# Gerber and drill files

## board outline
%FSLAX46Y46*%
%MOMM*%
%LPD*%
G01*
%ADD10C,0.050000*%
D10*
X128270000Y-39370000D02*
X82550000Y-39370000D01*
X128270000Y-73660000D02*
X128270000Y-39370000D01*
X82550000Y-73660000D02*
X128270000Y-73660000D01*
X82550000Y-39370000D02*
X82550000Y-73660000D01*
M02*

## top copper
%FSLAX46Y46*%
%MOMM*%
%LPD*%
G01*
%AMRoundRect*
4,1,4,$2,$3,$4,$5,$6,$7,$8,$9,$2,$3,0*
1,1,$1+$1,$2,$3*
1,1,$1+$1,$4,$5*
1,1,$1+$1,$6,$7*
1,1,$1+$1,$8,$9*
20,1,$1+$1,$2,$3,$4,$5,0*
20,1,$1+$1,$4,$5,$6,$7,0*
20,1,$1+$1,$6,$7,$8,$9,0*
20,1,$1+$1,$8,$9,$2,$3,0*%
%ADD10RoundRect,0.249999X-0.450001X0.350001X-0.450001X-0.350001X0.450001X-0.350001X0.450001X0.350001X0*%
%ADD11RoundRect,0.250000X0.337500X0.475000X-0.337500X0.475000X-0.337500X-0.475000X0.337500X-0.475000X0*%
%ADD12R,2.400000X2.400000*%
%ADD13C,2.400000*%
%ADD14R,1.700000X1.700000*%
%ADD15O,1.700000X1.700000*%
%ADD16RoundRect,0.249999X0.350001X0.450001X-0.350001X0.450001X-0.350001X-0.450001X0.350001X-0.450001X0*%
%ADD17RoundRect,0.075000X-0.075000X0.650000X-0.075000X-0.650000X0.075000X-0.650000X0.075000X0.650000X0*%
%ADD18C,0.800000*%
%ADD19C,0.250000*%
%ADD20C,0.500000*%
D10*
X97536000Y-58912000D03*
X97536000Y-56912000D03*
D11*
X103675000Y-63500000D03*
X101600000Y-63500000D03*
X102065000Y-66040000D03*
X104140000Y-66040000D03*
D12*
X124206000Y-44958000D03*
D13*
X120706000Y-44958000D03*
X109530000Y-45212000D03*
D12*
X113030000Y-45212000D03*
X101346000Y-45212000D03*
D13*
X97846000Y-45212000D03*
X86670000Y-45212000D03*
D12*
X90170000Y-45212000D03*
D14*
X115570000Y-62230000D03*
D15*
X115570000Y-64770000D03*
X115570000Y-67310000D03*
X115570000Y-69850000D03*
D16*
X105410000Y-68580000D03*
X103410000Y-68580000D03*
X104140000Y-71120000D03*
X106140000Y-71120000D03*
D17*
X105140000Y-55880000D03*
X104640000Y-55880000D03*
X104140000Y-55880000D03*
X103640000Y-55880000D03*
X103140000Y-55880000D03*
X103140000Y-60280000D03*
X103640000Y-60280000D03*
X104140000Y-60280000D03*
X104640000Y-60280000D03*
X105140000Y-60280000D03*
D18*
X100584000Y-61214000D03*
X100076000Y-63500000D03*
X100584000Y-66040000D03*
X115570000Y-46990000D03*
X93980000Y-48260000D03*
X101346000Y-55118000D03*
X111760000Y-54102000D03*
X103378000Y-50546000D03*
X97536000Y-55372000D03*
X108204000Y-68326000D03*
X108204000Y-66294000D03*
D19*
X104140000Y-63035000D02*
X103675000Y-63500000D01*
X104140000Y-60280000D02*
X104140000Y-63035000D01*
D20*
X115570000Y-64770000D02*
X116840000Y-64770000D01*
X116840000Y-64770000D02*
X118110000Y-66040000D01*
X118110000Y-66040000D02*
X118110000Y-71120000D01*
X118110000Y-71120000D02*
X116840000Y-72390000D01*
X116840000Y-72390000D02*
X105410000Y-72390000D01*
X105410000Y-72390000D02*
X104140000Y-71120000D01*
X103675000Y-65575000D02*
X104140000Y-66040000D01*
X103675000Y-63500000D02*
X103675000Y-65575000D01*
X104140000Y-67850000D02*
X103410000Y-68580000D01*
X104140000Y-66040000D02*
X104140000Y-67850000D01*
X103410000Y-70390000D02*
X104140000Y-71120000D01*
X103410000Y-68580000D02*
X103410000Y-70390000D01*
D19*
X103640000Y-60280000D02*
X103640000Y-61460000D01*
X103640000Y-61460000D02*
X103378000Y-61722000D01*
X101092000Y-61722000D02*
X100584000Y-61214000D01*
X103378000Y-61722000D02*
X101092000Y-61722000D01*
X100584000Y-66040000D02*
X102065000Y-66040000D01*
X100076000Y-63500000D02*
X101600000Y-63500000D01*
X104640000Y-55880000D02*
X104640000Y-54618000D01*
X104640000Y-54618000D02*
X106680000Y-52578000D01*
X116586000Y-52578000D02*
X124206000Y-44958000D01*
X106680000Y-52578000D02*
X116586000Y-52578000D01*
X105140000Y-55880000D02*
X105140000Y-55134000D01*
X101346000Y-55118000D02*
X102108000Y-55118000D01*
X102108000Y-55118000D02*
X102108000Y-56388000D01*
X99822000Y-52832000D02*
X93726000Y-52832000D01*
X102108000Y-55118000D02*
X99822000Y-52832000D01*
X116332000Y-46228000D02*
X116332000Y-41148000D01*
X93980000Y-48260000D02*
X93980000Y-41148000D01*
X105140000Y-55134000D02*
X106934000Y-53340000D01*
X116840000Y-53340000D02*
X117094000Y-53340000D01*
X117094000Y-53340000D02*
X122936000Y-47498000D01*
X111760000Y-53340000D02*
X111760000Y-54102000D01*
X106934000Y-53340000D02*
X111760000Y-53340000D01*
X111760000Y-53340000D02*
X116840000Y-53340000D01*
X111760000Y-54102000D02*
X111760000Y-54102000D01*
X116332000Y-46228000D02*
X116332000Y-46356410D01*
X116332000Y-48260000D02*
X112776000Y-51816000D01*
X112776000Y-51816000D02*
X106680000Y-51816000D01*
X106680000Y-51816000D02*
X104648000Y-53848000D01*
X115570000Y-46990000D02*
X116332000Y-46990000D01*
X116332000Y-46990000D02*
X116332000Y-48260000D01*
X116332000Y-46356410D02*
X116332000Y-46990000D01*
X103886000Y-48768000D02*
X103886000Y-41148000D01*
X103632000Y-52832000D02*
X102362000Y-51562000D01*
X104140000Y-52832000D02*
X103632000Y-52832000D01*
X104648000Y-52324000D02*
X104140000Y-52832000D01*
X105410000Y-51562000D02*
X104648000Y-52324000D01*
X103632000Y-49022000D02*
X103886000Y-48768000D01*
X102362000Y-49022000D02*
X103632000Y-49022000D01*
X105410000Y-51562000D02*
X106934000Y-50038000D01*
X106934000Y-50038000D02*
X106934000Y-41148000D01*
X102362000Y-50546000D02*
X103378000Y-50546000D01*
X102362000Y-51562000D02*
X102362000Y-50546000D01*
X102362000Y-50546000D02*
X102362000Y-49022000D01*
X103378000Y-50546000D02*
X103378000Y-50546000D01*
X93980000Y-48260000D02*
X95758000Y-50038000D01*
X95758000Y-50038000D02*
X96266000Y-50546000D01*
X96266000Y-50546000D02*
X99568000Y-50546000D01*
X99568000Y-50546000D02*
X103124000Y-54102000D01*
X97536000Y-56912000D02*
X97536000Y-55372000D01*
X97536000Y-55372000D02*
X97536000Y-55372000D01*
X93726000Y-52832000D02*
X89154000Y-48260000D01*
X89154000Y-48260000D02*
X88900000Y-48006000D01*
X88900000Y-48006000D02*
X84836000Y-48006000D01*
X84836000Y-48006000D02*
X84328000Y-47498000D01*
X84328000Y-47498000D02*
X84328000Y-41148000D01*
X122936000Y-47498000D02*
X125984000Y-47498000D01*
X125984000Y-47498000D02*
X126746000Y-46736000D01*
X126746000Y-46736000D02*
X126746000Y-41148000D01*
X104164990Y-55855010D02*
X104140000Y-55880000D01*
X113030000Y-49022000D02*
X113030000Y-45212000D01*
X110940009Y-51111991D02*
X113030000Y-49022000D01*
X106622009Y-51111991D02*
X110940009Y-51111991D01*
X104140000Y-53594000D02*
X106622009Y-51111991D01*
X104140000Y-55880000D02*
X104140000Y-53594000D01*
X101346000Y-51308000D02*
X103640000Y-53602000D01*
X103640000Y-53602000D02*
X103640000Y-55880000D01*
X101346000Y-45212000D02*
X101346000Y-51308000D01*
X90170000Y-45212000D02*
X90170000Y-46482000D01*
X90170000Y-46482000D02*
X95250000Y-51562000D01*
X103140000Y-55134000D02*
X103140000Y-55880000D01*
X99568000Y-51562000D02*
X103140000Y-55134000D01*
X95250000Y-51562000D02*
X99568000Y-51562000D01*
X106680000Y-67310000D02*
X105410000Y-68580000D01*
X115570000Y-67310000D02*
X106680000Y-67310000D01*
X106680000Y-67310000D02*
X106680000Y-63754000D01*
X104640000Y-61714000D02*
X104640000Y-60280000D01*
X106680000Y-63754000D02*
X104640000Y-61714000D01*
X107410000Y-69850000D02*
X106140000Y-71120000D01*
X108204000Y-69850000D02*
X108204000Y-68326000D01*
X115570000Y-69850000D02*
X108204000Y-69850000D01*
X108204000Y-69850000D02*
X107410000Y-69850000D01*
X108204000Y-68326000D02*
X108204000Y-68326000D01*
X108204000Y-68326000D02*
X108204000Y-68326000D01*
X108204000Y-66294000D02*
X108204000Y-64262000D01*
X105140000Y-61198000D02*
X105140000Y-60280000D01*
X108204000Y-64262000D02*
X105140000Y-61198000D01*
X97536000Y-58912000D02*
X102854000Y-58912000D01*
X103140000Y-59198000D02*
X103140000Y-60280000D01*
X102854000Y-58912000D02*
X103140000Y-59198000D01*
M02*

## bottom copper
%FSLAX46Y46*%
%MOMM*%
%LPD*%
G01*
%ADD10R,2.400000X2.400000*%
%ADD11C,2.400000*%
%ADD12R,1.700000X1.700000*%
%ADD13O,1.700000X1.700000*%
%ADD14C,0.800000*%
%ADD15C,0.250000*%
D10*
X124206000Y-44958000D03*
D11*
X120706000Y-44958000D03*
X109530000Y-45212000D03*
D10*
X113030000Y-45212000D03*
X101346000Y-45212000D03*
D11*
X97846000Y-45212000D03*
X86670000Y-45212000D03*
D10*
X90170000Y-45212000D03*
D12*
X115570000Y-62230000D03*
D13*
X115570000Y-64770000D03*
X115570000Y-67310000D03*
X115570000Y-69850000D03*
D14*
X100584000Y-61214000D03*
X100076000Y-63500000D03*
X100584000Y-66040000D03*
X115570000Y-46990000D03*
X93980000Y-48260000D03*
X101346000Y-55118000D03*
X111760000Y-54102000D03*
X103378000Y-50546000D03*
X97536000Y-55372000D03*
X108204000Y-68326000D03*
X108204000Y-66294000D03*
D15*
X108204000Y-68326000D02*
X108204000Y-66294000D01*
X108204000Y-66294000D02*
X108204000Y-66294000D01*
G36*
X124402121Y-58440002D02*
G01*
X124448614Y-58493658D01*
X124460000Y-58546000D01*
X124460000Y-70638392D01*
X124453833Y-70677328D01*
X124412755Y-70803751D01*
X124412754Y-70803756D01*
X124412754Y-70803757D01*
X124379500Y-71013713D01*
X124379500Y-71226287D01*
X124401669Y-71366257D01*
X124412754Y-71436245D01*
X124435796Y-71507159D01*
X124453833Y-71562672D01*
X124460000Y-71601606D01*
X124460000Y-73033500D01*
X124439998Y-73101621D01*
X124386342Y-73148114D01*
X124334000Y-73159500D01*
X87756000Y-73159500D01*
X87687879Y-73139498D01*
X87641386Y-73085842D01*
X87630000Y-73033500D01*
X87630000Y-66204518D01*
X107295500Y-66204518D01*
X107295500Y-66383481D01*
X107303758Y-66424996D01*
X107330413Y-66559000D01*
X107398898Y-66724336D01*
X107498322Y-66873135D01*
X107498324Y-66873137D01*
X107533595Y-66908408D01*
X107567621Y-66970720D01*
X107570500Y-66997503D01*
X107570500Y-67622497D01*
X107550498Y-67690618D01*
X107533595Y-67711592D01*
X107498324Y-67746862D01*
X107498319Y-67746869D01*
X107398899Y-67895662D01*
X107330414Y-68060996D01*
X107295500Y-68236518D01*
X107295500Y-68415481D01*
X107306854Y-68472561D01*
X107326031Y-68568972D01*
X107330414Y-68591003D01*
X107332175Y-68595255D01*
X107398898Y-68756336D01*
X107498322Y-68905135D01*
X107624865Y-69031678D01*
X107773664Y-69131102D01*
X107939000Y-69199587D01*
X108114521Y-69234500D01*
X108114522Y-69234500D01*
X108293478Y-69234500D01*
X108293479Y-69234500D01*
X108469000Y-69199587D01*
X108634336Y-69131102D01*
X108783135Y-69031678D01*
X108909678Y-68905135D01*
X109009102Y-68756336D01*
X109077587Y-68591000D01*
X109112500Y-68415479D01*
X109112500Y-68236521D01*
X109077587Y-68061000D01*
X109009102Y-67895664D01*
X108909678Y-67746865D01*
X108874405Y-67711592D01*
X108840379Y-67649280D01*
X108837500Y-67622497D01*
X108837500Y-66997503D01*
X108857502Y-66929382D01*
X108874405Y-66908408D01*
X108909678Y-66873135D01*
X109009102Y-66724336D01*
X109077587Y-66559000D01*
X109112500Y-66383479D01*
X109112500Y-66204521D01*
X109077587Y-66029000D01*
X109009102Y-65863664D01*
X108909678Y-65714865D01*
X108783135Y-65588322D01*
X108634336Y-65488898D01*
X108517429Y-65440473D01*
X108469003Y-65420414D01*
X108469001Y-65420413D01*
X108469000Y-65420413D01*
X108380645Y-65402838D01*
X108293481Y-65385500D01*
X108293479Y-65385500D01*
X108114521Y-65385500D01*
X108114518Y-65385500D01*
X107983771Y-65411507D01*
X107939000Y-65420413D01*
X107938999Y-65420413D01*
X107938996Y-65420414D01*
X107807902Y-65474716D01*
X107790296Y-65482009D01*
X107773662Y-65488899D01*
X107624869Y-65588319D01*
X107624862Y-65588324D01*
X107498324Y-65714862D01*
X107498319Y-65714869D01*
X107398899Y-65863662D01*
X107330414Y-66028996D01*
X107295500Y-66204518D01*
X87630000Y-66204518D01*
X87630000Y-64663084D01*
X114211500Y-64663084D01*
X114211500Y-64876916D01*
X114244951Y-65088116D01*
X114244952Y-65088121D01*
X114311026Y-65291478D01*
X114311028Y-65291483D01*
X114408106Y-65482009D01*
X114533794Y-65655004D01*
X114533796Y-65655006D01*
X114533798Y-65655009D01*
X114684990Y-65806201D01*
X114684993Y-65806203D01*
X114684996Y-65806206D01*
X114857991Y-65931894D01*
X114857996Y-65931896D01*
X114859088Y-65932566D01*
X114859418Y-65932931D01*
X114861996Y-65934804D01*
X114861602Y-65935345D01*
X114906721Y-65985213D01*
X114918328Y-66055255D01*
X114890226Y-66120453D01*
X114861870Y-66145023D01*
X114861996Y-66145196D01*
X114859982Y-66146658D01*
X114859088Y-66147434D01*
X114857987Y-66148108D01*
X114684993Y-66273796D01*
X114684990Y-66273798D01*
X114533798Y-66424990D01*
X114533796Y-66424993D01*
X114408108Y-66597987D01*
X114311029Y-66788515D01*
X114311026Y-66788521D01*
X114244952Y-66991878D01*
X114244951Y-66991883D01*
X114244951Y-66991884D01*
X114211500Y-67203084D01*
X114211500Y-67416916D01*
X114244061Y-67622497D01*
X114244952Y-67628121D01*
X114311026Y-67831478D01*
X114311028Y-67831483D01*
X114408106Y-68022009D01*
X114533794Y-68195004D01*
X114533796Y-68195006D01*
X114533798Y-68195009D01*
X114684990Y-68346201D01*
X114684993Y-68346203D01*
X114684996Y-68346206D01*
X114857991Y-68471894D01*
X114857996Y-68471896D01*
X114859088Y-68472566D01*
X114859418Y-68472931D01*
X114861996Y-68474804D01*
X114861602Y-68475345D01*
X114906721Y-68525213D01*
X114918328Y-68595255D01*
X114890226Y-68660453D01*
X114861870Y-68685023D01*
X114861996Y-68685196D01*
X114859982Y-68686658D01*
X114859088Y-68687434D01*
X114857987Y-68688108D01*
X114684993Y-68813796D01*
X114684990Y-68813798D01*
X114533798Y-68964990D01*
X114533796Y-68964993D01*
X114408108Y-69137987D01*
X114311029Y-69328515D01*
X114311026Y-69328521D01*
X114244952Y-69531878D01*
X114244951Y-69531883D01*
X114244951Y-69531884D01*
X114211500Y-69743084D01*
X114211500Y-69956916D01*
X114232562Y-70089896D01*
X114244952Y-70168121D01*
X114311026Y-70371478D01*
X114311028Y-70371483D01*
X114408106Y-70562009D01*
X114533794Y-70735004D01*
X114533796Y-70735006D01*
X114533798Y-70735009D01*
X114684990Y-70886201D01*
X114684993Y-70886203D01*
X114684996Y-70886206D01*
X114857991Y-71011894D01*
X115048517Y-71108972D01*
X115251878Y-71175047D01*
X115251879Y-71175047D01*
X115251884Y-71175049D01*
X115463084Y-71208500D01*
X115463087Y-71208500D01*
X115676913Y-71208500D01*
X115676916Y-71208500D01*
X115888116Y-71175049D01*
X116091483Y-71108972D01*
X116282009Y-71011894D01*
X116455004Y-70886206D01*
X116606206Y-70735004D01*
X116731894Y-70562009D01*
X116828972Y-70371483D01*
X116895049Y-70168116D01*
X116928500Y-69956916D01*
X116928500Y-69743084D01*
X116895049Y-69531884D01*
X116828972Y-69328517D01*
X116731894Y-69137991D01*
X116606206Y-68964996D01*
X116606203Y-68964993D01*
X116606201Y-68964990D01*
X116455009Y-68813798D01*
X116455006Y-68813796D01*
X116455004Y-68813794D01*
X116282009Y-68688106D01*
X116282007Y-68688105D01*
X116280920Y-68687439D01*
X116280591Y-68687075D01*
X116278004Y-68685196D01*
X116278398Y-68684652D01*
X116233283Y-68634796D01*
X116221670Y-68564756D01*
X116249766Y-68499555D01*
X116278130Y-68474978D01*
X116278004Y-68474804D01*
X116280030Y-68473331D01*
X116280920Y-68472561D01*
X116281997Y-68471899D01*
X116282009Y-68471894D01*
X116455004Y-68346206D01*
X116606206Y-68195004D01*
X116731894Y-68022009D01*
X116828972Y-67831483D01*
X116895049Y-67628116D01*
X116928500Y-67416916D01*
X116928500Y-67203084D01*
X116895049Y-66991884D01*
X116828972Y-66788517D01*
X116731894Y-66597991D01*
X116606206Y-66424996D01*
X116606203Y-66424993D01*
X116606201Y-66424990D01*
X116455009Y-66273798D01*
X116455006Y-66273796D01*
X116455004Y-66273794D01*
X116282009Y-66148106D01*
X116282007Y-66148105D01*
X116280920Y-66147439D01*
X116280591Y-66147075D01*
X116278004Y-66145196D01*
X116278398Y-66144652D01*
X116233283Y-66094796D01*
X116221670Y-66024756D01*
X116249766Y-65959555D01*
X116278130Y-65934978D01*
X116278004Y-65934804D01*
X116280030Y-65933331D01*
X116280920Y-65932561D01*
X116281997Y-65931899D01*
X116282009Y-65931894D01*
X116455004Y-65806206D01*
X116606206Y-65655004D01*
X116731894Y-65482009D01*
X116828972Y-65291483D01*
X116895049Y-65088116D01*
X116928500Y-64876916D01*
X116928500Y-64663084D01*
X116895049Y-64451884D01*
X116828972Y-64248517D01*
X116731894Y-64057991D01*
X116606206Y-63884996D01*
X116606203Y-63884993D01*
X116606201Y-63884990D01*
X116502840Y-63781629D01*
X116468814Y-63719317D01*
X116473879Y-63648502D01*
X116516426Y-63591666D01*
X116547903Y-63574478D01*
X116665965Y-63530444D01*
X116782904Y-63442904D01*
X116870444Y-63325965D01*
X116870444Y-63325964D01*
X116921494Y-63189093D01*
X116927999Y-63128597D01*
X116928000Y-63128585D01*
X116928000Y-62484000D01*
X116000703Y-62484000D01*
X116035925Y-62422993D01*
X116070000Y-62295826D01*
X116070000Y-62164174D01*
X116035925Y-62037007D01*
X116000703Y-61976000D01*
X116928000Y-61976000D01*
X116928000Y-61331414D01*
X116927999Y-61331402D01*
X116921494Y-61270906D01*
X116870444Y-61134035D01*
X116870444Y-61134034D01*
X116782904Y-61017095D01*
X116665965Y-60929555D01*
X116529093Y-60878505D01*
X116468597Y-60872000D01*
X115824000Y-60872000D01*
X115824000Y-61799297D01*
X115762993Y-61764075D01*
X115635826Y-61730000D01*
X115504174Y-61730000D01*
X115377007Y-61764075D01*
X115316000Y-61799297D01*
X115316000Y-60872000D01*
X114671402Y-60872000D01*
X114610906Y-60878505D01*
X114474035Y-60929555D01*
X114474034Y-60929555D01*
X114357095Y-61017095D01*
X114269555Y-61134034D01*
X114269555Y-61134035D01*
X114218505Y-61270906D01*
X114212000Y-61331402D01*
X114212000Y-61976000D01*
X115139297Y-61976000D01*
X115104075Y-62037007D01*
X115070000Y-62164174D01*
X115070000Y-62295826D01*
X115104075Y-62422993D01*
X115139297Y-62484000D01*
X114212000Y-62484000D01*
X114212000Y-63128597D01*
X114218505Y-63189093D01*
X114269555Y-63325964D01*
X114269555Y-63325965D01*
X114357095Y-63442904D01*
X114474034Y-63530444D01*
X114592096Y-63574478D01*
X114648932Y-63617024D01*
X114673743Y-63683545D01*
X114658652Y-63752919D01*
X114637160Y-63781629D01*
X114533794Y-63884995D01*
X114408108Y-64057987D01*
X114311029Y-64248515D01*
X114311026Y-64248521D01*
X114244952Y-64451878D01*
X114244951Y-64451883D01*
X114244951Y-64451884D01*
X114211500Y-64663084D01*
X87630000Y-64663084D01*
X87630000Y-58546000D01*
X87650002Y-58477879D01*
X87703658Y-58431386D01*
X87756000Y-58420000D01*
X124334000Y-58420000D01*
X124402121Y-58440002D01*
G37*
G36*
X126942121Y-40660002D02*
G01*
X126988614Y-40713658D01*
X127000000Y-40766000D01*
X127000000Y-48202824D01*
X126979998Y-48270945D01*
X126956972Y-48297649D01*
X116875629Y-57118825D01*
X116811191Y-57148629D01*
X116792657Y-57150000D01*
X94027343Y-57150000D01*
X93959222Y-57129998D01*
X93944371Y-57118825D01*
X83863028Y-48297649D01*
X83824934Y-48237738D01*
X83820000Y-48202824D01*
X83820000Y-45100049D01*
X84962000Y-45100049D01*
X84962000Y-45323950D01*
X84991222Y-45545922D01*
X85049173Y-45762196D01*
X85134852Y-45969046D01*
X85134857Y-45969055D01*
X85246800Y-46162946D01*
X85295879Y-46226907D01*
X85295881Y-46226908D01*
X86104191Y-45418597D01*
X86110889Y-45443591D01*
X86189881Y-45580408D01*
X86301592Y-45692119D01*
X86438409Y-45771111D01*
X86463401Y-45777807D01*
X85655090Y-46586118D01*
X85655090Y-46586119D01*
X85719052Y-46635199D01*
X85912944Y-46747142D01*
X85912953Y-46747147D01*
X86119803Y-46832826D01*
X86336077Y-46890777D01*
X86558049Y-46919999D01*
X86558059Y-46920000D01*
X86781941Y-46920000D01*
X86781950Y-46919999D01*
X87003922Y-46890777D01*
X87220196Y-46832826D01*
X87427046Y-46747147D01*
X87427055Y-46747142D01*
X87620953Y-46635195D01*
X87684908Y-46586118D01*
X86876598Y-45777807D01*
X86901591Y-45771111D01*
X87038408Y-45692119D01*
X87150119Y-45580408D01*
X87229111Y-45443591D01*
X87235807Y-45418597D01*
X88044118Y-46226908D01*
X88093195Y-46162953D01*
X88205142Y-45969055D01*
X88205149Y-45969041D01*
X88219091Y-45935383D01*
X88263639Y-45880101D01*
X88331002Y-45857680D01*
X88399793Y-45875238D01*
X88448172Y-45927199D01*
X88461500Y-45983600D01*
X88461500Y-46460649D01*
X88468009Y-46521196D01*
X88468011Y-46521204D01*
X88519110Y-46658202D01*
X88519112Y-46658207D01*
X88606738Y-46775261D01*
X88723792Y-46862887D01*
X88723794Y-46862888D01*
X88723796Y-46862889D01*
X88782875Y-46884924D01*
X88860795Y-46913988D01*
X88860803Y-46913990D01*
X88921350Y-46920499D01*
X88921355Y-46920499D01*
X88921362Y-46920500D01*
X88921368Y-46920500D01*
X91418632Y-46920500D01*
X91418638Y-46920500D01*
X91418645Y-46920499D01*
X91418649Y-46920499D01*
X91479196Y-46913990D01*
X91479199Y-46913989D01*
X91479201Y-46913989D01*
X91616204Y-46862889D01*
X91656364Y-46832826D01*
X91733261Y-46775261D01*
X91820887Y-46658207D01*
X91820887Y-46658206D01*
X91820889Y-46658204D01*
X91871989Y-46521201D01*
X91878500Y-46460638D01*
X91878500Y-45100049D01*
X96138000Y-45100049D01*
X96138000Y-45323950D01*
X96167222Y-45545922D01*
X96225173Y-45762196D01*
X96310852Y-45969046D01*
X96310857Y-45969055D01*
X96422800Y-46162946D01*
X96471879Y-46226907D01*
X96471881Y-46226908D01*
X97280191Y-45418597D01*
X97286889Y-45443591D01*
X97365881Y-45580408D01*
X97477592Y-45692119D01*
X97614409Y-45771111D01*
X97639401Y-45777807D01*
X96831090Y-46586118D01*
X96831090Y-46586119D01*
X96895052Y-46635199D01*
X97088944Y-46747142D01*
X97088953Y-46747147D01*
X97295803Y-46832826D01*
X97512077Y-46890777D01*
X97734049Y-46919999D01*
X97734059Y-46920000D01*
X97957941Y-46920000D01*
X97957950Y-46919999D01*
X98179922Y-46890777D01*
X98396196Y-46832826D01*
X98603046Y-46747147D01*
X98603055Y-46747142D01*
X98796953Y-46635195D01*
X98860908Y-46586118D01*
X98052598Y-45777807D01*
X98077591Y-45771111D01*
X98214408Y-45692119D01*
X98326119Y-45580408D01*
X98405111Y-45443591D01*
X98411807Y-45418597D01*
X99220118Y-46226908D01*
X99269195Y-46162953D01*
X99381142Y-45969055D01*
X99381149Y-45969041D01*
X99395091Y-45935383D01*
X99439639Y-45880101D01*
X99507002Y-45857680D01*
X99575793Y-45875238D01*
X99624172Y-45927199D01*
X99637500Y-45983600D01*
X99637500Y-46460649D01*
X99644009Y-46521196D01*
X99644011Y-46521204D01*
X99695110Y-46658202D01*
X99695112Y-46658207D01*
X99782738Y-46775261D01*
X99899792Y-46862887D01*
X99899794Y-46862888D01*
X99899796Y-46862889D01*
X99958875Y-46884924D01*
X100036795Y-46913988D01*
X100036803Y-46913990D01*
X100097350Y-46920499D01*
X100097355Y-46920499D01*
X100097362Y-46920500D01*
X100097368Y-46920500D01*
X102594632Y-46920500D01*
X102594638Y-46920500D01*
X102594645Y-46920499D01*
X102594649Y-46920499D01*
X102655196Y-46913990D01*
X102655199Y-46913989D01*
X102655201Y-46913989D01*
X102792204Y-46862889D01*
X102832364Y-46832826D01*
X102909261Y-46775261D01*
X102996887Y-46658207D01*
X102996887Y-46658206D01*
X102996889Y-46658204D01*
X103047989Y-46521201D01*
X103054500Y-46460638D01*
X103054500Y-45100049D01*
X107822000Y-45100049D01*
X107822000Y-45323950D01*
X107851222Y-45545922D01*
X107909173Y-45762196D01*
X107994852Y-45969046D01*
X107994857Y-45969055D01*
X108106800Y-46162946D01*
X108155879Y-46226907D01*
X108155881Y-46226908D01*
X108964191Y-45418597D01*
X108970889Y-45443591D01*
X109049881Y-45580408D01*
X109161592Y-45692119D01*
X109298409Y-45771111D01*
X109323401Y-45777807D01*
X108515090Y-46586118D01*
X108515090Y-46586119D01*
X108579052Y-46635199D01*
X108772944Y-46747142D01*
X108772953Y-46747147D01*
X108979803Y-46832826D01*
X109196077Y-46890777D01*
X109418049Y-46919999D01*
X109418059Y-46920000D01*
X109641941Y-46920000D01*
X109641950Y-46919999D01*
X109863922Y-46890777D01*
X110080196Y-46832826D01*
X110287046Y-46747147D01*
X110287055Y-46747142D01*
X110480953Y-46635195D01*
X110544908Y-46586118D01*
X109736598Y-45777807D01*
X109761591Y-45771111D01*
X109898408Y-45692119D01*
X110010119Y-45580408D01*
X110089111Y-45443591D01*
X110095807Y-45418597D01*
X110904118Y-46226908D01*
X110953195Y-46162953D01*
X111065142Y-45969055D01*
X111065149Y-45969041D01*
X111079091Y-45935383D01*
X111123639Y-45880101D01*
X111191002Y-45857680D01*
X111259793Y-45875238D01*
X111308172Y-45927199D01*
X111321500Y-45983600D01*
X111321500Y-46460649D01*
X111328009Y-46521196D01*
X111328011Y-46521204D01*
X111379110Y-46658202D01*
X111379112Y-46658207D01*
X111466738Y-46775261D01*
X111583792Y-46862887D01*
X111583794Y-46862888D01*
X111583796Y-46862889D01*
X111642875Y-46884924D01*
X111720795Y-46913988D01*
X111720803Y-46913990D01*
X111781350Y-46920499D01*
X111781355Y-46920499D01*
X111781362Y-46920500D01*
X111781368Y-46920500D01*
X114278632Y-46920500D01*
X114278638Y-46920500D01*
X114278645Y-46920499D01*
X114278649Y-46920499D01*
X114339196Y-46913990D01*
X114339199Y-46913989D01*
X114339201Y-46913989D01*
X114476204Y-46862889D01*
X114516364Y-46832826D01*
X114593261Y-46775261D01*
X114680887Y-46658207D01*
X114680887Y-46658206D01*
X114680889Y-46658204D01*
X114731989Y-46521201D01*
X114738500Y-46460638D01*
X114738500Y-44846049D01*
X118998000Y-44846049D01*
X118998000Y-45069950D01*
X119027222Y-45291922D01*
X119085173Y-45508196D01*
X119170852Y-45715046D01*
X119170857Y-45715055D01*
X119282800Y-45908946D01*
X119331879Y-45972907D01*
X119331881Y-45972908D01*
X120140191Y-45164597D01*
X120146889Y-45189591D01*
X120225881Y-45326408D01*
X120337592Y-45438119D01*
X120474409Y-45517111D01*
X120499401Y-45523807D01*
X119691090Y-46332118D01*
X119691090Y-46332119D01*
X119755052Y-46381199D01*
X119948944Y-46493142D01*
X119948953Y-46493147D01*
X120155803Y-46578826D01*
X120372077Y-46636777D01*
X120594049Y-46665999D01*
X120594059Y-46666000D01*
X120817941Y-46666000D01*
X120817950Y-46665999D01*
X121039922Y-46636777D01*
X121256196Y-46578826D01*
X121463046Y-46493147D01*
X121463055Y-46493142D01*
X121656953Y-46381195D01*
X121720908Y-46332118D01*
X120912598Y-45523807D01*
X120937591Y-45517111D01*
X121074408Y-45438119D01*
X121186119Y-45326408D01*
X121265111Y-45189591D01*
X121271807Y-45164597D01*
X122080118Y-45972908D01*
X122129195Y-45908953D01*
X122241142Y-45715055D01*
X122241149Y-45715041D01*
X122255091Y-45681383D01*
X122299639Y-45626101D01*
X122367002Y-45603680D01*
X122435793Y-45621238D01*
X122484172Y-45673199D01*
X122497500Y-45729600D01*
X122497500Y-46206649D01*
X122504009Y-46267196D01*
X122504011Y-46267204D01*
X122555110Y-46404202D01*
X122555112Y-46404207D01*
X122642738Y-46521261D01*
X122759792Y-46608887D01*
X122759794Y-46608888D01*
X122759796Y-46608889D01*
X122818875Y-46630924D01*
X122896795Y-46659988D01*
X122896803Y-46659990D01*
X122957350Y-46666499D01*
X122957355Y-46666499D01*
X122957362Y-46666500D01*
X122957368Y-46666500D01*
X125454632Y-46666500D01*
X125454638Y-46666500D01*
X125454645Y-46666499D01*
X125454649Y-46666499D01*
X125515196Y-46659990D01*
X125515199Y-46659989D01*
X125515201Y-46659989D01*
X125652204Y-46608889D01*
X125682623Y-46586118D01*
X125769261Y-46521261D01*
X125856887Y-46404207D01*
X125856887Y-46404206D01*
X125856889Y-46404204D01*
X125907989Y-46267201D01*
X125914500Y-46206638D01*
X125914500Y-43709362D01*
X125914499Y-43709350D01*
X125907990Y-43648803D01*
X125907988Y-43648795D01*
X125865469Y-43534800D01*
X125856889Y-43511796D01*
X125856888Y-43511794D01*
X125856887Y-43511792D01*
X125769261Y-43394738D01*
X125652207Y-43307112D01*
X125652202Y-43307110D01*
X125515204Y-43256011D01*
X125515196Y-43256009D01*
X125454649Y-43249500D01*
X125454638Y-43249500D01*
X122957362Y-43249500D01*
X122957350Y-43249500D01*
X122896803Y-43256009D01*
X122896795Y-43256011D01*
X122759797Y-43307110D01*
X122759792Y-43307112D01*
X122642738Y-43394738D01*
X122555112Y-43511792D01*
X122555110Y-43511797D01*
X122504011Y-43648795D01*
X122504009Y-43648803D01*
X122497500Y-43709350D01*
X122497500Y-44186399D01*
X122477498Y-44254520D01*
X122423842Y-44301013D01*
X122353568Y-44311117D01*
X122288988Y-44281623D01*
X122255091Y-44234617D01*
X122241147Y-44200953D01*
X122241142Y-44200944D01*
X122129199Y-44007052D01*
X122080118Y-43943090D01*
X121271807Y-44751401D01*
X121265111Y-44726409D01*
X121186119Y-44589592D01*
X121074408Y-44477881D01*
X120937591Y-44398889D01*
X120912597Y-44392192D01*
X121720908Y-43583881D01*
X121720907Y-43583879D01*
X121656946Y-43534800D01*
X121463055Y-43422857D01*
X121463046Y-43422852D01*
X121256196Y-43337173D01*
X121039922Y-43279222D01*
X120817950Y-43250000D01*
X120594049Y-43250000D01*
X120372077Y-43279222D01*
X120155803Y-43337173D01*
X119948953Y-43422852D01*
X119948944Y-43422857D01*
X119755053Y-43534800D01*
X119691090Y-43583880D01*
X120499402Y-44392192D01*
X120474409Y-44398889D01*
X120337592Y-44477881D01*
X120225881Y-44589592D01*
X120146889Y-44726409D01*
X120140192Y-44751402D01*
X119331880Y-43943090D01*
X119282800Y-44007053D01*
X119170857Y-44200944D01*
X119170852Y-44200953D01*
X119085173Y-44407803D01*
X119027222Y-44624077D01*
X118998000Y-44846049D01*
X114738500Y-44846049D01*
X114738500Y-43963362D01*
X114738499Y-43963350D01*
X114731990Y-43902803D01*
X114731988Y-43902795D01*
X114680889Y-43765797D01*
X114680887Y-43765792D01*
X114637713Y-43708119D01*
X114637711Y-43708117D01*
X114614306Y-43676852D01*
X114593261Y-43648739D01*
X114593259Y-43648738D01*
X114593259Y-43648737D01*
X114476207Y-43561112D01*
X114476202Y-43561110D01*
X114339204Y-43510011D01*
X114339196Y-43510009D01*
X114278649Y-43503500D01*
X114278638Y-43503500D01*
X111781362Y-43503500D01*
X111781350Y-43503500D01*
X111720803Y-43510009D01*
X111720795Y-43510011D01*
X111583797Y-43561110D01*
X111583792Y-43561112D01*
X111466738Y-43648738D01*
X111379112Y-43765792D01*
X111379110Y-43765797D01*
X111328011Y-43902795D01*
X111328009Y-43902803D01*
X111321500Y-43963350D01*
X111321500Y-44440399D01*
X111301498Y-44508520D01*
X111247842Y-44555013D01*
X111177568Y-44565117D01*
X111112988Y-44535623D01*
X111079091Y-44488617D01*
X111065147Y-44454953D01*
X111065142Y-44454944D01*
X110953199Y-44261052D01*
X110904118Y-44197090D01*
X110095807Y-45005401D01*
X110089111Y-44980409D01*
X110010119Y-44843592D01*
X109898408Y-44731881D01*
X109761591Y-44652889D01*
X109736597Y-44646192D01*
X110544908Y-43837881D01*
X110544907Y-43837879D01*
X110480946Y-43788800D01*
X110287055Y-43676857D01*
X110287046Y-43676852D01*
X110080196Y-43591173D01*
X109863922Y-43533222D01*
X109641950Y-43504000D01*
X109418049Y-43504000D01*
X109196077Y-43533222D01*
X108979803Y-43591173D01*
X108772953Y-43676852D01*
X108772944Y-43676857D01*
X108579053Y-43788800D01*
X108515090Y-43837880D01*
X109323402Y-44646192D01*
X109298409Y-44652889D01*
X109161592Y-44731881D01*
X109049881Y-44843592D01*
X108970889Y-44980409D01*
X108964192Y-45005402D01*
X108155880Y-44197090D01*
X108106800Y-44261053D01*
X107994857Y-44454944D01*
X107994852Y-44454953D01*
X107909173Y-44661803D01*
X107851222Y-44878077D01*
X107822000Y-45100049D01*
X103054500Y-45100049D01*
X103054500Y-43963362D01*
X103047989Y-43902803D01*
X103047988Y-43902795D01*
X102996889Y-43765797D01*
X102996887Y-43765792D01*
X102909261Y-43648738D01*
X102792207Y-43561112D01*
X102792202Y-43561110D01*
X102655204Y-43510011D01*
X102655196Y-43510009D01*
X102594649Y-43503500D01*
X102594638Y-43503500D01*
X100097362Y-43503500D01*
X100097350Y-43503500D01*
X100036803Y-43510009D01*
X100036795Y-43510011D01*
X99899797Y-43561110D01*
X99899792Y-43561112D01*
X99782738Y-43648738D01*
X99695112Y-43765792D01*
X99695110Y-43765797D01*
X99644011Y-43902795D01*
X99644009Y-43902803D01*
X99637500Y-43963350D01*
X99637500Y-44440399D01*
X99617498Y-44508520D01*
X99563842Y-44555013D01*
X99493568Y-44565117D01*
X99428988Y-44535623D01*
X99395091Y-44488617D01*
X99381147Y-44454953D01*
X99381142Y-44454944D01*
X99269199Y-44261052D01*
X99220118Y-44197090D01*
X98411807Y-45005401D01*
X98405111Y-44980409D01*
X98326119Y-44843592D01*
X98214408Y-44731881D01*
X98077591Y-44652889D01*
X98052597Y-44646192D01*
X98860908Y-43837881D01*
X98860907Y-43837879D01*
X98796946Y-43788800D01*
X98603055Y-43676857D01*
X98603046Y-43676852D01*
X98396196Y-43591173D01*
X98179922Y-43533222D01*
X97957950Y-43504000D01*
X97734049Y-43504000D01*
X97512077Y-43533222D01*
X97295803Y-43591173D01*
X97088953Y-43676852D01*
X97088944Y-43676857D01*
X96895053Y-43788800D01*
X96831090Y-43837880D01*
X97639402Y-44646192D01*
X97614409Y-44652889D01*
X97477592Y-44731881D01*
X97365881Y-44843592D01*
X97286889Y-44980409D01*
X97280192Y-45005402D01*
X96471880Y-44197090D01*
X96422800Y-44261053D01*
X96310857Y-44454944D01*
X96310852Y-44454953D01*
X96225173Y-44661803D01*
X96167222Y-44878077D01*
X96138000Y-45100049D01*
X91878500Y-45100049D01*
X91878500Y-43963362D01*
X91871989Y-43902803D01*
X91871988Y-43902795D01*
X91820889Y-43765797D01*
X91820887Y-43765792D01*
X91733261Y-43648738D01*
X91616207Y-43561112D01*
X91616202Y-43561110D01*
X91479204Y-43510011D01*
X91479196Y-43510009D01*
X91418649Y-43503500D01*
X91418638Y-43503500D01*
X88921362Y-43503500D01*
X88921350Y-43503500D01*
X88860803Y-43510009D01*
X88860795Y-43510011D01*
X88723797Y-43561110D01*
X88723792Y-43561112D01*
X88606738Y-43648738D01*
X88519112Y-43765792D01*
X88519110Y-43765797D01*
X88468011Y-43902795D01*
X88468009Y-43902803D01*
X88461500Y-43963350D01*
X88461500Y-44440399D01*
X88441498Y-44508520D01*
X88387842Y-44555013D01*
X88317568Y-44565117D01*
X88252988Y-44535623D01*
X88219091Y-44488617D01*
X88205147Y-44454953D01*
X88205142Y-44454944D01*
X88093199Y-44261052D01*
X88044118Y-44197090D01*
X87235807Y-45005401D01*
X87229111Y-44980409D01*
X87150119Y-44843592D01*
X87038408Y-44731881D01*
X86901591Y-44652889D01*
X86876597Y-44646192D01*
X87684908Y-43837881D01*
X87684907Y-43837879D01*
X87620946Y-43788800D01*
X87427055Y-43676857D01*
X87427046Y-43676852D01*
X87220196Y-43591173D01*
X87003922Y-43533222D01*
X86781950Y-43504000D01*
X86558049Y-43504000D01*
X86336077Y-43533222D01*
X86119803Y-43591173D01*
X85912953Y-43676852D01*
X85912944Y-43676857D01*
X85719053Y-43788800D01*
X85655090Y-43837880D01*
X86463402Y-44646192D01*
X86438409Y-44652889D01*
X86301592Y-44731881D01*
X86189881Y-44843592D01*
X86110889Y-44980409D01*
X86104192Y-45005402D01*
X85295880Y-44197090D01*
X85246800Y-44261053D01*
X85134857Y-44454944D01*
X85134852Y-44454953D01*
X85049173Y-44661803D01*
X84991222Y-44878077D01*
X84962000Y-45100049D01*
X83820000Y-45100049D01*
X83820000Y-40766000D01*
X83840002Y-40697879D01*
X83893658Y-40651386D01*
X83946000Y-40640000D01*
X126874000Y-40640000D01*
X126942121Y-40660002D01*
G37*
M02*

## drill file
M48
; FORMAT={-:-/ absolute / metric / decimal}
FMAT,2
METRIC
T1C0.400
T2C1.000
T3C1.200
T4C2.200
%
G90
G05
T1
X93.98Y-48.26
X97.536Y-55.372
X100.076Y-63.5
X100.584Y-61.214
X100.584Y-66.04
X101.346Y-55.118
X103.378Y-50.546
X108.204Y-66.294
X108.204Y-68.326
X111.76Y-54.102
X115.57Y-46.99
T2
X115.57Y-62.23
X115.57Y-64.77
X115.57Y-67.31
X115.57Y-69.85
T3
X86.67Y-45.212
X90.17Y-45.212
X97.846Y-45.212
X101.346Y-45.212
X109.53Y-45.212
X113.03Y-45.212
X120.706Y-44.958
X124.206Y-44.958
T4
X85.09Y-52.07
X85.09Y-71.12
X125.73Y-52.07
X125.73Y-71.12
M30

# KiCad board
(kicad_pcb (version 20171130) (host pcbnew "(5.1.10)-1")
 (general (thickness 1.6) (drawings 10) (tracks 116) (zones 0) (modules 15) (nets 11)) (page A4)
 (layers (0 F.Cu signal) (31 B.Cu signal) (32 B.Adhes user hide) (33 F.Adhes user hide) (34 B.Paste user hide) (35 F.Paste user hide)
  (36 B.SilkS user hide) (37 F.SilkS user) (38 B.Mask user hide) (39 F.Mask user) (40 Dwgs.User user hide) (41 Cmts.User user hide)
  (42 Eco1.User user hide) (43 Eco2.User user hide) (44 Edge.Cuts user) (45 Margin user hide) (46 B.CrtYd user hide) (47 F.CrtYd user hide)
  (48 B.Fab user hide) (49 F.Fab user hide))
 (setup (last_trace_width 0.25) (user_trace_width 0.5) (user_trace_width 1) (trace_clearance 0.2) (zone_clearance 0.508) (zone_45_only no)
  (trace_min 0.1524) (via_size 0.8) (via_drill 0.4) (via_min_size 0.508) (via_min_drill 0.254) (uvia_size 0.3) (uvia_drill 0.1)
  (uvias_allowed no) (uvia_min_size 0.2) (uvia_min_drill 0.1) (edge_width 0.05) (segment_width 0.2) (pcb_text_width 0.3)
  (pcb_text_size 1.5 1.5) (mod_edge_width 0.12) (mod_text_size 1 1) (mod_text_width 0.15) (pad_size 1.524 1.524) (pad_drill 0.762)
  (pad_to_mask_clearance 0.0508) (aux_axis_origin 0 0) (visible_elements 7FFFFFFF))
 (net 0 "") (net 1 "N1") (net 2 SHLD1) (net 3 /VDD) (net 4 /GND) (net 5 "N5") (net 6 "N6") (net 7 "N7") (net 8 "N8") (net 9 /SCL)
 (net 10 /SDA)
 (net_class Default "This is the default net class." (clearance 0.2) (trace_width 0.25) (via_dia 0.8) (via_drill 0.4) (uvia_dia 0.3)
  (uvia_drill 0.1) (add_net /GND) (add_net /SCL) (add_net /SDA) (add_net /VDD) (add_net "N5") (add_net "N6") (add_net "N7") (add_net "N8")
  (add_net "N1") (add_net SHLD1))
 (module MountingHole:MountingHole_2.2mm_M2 (layer F.Cu) (at 125.73 71.12)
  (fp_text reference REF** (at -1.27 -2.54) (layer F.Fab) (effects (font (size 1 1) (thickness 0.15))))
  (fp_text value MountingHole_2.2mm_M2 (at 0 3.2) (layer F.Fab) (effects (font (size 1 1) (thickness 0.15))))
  (pad 1 np_thru_hole circle (at 0 0) (size 2.2 2.2) (drill 2.2) (layers *.Cu *.Mask)))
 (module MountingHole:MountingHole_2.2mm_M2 (layer F.Cu) (at 85.09 71.12)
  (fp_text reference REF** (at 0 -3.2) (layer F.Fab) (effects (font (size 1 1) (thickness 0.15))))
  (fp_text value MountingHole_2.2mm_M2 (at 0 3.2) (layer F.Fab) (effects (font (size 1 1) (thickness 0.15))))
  (pad 1 np_thru_hole circle (at 0 0) (size 2.2 2.2) (drill 2.2) (layers *.Cu *.Mask)))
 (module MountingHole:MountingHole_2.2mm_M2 (layer F.Cu) (at 85.09 52.07)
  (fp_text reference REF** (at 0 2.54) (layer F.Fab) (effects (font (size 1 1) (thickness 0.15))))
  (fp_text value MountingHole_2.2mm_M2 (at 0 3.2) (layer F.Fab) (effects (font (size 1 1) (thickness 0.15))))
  (pad 1 np_thru_hole circle (at 0 0) (size 2.2 2.2) (drill 2.2) (layers *.Cu *.Mask)))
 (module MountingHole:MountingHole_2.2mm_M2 (layer F.Cu) (at 125.73 52.07)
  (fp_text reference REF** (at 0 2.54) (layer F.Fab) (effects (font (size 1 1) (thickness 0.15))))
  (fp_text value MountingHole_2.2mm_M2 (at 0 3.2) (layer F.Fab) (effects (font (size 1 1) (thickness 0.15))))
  (pad 1 np_thru_hole circle (at 0 0) (size 2.2 2.2) (drill 2.2) (layers *.Cu *.Mask)))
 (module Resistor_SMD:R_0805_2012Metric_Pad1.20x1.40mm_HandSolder (layer F.Cu) (at 97.536 57.912 270)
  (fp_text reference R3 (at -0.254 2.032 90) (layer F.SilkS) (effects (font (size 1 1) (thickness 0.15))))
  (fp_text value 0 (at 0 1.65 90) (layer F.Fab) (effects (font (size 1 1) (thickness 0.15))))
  (pad 2 smd roundrect (at 1 0 270) (size 1.2 1.4) (layers F.Cu F.Paste F.Mask) (roundrect_rratio 0.2083325) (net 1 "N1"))
  (pad 1 smd roundrect (at -1 0 270) (size 1.2 1.4) (layers F.Cu F.Paste F.Mask) (roundrect_rratio 0.2083325) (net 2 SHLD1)))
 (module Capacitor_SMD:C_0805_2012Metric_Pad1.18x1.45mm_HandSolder (layer F.Cu) (at 102.6375 63.5 180)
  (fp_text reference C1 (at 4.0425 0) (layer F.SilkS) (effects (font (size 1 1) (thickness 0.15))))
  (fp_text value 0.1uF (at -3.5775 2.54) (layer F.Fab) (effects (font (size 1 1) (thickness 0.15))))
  (pad 1 smd roundrect (at -1.0375 0 180) (size 1.175 1.45) (layers F.Cu F.Paste F.Mask) (roundrect_rratio 0.2127659574468085) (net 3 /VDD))
  (pad 2 smd roundrect (at 1.0375 0 180) (size 1.175 1.45) (layers F.Cu F.Paste F.Mask) (roundrect_rratio 0.2127659574468085) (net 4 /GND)))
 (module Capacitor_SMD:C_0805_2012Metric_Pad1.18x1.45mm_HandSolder (layer F.Cu) (at 103.1025 66.04 180)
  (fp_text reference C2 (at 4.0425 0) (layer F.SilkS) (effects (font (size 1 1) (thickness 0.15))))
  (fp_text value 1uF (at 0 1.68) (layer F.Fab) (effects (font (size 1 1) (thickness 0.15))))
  (pad 2 smd roundrect (at 1.0375 0 180) (size 1.175 1.45) (layers F.Cu F.Paste F.Mask) (roundrect_rratio 0.2127659574468085) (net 4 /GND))
  (pad 1 smd roundrect (at -1.0375 0 180) (size 1.175 1.45) (layers F.Cu F.Paste F.Mask) (roundrect_rratio 0.2127659574468085) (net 3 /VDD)))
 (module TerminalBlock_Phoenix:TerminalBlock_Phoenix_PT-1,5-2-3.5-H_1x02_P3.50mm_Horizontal (layer F.Cu) (at 124.206 44.958 180)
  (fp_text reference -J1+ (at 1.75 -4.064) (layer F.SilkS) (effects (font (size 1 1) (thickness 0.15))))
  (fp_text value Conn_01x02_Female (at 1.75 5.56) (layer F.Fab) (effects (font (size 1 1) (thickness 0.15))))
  (pad 1 thru_hole rect (at 0 0 180) (size 2.4 2.4) (drill 1.2) (layers *.Cu *.Mask) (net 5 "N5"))
  (pad 2 thru_hole circle (at 3.5 0 180) (size 2.4 2.4) (drill 1.2) (layers *.Cu *.Mask) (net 2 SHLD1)))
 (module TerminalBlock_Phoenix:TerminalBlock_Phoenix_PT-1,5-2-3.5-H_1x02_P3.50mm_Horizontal (layer F.Cu) (at 113.03 45.212 180)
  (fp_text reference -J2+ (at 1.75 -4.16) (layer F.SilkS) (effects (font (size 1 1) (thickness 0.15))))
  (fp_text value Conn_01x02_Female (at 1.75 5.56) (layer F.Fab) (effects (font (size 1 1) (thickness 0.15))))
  (pad 2 thru_hole circle (at 3.5 0 180) (size 2.4 2.4) (drill 1.2) (layers *.Cu *.Mask) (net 2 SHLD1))
  (pad 1 thru_hole rect (at 0 0 180) (size 2.4 2.4) (drill 1.2) (layers *.Cu *.Mask) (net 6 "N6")))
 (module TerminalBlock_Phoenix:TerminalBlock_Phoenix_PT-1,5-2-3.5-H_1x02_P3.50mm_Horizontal (layer F.Cu) (at 101.346 45.212 180)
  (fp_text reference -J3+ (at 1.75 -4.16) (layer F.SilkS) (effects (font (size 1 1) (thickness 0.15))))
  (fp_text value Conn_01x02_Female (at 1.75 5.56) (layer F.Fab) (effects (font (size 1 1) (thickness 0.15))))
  (pad 1 thru_hole rect (at 0 0 180) (size 2.4 2.4) (drill 1.2) (layers *.Cu *.Mask) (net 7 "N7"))
  (pad 2 thru_hole circle (at 3.5 0 180) (size 2.4 2.4) (drill 1.2) (layers *.Cu *.Mask) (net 2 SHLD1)))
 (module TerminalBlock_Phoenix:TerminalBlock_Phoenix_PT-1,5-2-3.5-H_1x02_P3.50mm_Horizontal (layer F.Cu) (at 90.17 45.212 180)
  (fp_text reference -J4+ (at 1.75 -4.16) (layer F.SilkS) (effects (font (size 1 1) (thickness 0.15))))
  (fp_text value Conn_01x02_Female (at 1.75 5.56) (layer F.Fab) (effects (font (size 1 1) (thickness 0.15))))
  (pad 2 thru_hole circle (at 3.5 0 180) (size 2.4 2.4) (drill 1.2) (layers *.Cu *.Mask) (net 2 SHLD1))
  (pad 1 thru_hole rect (at 0 0 180) (size 2.4 2.4) (drill 1.2) (layers *.Cu *.Mask) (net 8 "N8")))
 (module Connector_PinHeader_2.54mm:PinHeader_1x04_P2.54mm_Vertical (layer F.Cu) (at 115.57 62.23)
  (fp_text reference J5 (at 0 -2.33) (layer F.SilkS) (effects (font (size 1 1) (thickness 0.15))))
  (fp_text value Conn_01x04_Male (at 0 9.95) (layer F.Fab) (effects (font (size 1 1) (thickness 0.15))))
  (pad 1 thru_hole rect (at 0 0) (size 1.7 1.7) (drill 1) (layers *.Cu *.Mask) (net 4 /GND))
  (pad 2 thru_hole oval (at 0 2.54) (size 1.7 1.7) (drill 1) (layers *.Cu *.Mask) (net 3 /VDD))
  (pad 3 thru_hole oval (at 0 5.08) (size 1.7 1.7) (drill 1) (layers *.Cu *.Mask) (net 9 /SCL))
  (pad 4 thru_hole oval (at 0 7.62) (size 1.7 1.7) (drill 1) (layers *.Cu *.Mask) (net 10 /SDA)))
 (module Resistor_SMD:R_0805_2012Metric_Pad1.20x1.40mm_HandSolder (layer F.Cu) (at 104.41 68.58 180)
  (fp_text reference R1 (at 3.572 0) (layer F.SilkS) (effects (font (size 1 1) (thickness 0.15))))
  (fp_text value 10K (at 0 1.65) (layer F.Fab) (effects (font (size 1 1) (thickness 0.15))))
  (pad 1 smd roundrect (at -1 0 180) (size 1.2 1.4) (layers F.Cu F.Paste F.Mask) (roundrect_rratio 0.2083325) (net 9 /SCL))
  (pad 2 smd roundrect (at 1 0 180) (size 1.2 1.4) (layers F.Cu F.Paste F.Mask) (roundrect_rratio 0.2083325) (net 3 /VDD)))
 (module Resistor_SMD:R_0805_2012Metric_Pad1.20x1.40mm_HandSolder (layer F.Cu) (at 105.14 71.12 180)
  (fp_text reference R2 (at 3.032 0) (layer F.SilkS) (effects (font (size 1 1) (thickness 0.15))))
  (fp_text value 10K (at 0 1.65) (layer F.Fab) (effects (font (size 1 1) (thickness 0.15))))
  (pad 2 smd roundrect (at 1 0 180) (size 1.2 1.4) (layers F.Cu F.Paste F.Mask) (roundrect_rratio 0.2083325) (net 3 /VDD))
  (pad 1 smd roundrect (at -1 0 180) (size 1.2 1.4) (layers F.Cu F.Paste F.Mask) (roundrect_rratio 0.2083325) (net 10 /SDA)))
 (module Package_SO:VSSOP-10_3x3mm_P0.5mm (layer F.Cu) (at 104.14 58.08 270)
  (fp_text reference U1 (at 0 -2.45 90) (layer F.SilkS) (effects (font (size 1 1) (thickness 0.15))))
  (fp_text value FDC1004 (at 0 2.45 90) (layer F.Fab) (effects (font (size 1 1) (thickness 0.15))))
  (pad 1 smd roundrect (at -2.2 -1 270) (size 1.45 0.3) (layers F.Cu F.Paste F.Mask) (roundrect_rratio 0.25) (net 2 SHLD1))
  (pad 2 smd roundrect (at -2.2 -0.5 270) (size 1.45 0.3) (layers F.Cu F.Paste F.Mask) (roundrect_rratio 0.25) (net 5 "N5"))
  (pad 3 smd roundrect (at -2.2 0 270) (size 1.45 0.3) (layers F.Cu F.Paste F.Mask) (roundrect_rratio 0.25) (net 6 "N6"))
  (pad 4 smd roundrect (at -2.2 0.5 270) (size 1.45 0.3) (layers F.Cu F.Paste F.Mask) (roundrect_rratio 0.25) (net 7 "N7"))
  (pad 5 smd roundrect (at -2.2 1 270) (size 1.45 0.3) (layers F.Cu F.Paste F.Mask) (roundrect_rratio 0.25) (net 8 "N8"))
  (pad 6 smd roundrect (at 2.2 1 270) (size 1.45 0.3) (layers F.Cu F.Paste F.Mask) (roundrect_rratio 0.25) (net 1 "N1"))
  (pad 7 smd roundrect (at 2.2 0.5 270) (size 1.45 0.3) (layers F.Cu F.Paste F.Mask) (roundrect_rratio 0.25) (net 4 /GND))
  (pad 8 smd roundrect (at 2.2 0 270) (size 1.45 0.3) (layers F.Cu F.Paste F.Mask) (roundrect_rratio 0.25) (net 3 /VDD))
  (pad 9 smd roundrect (at 2.2 -0.5 270) (size 1.45 0.3) (layers F.Cu F.Paste F.Mask) (roundrect_rratio 0.25) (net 9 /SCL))
  (pad 10 smd roundrect (at 2.2 -1 270) (size 1.45 0.3) (layers F.Cu F.Paste F.Mask) (roundrect_rratio 0.25) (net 10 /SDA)))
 (gr_line (start 128.27 39.37) (end 82.55 39.37) (layer Edge.Cuts) (width 0.05))
 (gr_line (start 128.27 73.66) (end 128.27 39.37) (layer Edge.Cuts) (width 0.05))
 (gr_line (start 82.55 73.66) (end 128.27 73.66) (layer Edge.Cuts) (width 0.05))
 (gr_line (start 82.55 39.37) (end 82.55 73.66) (layer Edge.Cuts) (width 0.05))
 (segment (start 104.14 63.035) (end 103.675 63.5) (width 0.25) (layer F.Cu) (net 3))
 (segment (start 104.14 60.28) (end 104.14 63.035) (width 0.25) (layer F.Cu) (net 3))
 (segment (start 115.57 64.77) (end 116.84 64.77) (width 0.5) (layer F.Cu) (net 3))
 (segment (start 116.84 64.77) (end 118.11 66.04) (width 0.5) (layer F.Cu) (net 3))
 (segment (start 118.11 66.04) (end 118.11 71.12) (width 0.5) (layer F.Cu) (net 3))
 (segment (start 118.11 71.12) (end 116.84 72.39) (width 0.5) (layer F.Cu) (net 3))
 (segment (start 116.84 72.39) (end 105.41 72.39) (width 0.5) (layer F.Cu) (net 3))
 (segment (start 105.41 72.39) (end 104.14 71.12) (width 0.5) (layer F.Cu) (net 3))
 (segment (start 103.675 65.575) (end 104.14 66.04) (width 0.5) (layer F.Cu) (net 3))
 (segment (start 103.675 63.5) (end 103.675 65.575) (width 0.5) (layer F.Cu) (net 3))
 (segment (start 104.14 67.85) (end 103.41 68.58) (width 0.5) (layer F.Cu) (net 3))
 (segment (start 104.14 66.04) (end 104.14 67.85) (width 0.5) (layer F.Cu) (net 3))
 (segment (start 103.41 70.39) (end 104.14 71.12) (width 0.5) (layer F.Cu) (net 3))
 (segment (start 103.41 68.58) (end 103.41 70.39) (width 0.5) (layer F.Cu) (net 3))
 (via (at 100.584 61.214) (size 0.8) (drill 0.4) (layers F.Cu B.Cu) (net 4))
 (segment (start 103.64 60.28) (end 103.64 61.46) (width 0.25) (layer F.Cu) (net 4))
 (segment (start 103.64 61.46) (end 103.378 61.722) (width 0.25) (layer F.Cu) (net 4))
 (segment (start 101.092 61.722) (end 100.584 61.214) (width 0.25) (layer F.Cu) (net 4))
 (segment (start 103.378 61.722) (end 101.092 61.722) (width 0.25) (layer F.Cu) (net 4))
 (via (at 100.076 63.5) (size 0.8) (drill 0.4) (layers F.Cu B.Cu) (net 4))
 (via (at 100.584 66.04) (size 0.8) (drill 0.4) (layers F.Cu B.Cu) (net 4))
 (segment (start 100.584 66.04) (end 102.065 66.04) (width 0.25) (layer F.Cu) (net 4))
 (segment (start 100.076 63.5) (end 101.6 63.5) (width 0.25) (layer F.Cu) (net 4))
 (segment (start 104.64 55.88) (end 104.64 54.618) (width 0.25) (layer F.Cu) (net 5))
 (segment (start 104.64 54.618) (end 106.68 52.578) (width 0.25) (layer F.Cu) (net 5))
 (segment (start 116.586 52.578) (end 124.206 44.958) (width 0.25) (layer F.Cu) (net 5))
 (segment (start 106.68 52.578) (end 116.586 52.578) (width 0.25) (layer F.Cu) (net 5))
 (via (at 115.57 46.99) (size 0.8) (drill 0.4) (layers F.Cu B.Cu) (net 2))
 (via (at 93.98 48.26) (size 0.8) (drill 0.4) (layers F.Cu B.Cu) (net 2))
 (segment (start 105.14 55.88) (end 105.14 55.134) (width 0.25) (layer F.Cu) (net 2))
 (via (at 101.346 55.118) (size 0.8) (drill 0.4) (layers F.Cu B.Cu) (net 2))
 (segment (start 101.346 55.118) (end 102.108 55.118) (width 0.25) (layer F.Cu) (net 2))
 (segment (start 102.108 55.118) (end 102.108 56.388) (width 0.25) (layer F.Cu) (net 2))
 (segment (start 99.822 52.832) (end 93.726 52.832) (width 0.25) (layer F.Cu) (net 2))
 (segment (start 102.108 55.118) (end 99.822 52.832) (width 0.25) (layer F.Cu) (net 2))
 (segment (start 116.332 46.228) (end 116.332 41.148) (width 0.25) (layer F.Cu) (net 2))
 (segment (start 93.98 48.26) (end 93.98 41.148) (width 0.25) (layer F.Cu) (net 2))
 (segment (start 105.14 55.134) (end 106.934 53.34) (width 0.25) (layer F.Cu) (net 2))
 (segment (start 116.84 53.34) (end 117.094 53.34) (width 0.25) (layer F.Cu) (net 2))
 (segment (start 117.094 53.34) (end 122.936 47.498) (width 0.25) (layer F.Cu) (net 2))
 (segment (start 111.76 53.34) (end 111.76 54.102) (width 0.25) (layer F.Cu) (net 2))
 (segment (start 106.934 53.34) (end 111.76 53.34) (width 0.25) (layer F.Cu) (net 2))
 (segment (start 111.76 53.34) (end 116.84 53.34) (width 0.25) (layer F.Cu) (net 2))
 (segment (start 111.76 54.102) (end 111.76 54.102) (width 0.25) (layer F.Cu) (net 2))
 (via (at 111.76 54.102) (size 0.8) (drill 0.4) (layers F.Cu B.Cu) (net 2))
 (segment (start 116.332 46.228) (end 116.332 46.35641) (width 0.25) (layer F.Cu) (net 2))
 (segment (start 116.332 48.26) (end 112.776 51.816) (width 0.25) (layer F.Cu) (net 2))
 (segment (start 112.776 51.816) (end 106.68 51.816) (width 0.25) (layer F.Cu) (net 2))
 (segment (start 106.68 51.816) (end 104.648 53.848) (width 0.25) (layer F.Cu) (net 2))
 (segment (start 115.57 46.99) (end 116.332 46.99) (width 0.25) (layer F.Cu) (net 2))
 (segment (start 116.332 46.99) (end 116.332 48.26) (width 0.25) (layer F.Cu) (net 2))
 (segment (start 116.332 46.35641) (end 116.332 46.99) (width 0.25) (layer F.Cu) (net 2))
 (segment (start 103.886 48.768) (end 103.886 41.148) (width 0.25) (layer F.Cu) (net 2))
 (segment (start 103.632 52.832) (end 102.362 51.562) (width 0.25) (layer F.Cu) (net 2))
 (segment (start 104.14 52.832) (end 103.632 52.832) (width 0.25) (layer F.Cu) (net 2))
 (segment (start 104.648 52.324) (end 104.14 52.832) (width 0.25) (layer F.Cu) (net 2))
 (segment (start 105.41 51.562) (end 104.648 52.324) (width 0.25) (layer F.Cu) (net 2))
 (segment (start 103.632 49.022) (end 103.886 48.768) (width 0.25) (layer F.Cu) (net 2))
 (segment (start 102.362 49.022) (end 103.632 49.022) (width 0.25) (layer F.Cu) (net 2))
 (segment (start 105.41 51.562) (end 106.934 50.038) (width 0.25) (layer F.Cu) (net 2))
 (segment (start 106.934 50.038) (end 106.934 41.148) (width 0.25) (layer F.Cu) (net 2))
 (segment (start 102.362 50.546) (end 103.378 50.546) (width 0.25) (layer F.Cu) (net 2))
 (segment (start 102.362 51.562) (end 102.362 50.546) (width 0.25) (layer F.Cu) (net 2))
 (segment (start 102.362 50.546) (end 102.362 49.022) (width 0.25) (layer F.Cu) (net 2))
 (segment (start 103.378 50.546) (end 103.378 50.546) (width 0.25) (layer F.Cu) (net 2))
 (via (at 103.378 50.546) (size 0.8) (drill 0.4) (layers F.Cu B.Cu) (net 2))
 (segment (start 93.98 48.26) (end 95.758 50.038) (width 0.25) (layer F.Cu) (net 2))
 (segment (start 95.758 50.038) (end 96.266 50.546) (width 0.25) (layer F.Cu) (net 2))
 (segment (start 96.266 50.546) (end 99.568 50.546) (width 0.25) (layer F.Cu) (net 2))
 (segment (start 99.568 50.546) (end 103.124 54.102) (width 0.25) (layer F.Cu) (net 2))
 (segment (start 97.536 56.912) (end 97.536 55.372) (width 0.25) (layer F.Cu) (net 2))
 (segment (start 97.536 55.372) (end 97.536 55.372) (width 0.25) (layer F.Cu) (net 2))
 (via (at 97.536 55.372) (size 0.8) (drill 0.4) (layers F.Cu B.Cu) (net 2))
 (segment (start 93.726 52.832) (end 89.154 48.26) (width 0.25) (layer F.Cu) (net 2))
 (segment (start 89.154 48.26) (end 88.9 48.006) (width 0.25) (layer F.Cu) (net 2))
 (segment (start 88.9 48.006) (end 84.836 48.006) (width 0.25) (layer F.Cu) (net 2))
 (segment (start 84.836 48.006) (end 84.328 47.498) (width 0.25) (layer F.Cu) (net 2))
 (segment (start 84.328 47.498) (end 84.328 41.148) (width 0.25) (layer F.Cu) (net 2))
 (segment (start 122.936 47.498) (end 125.984 47.498) (width 0.25) (layer F.Cu) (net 2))
 (segment (start 125.984 47.498) (end 126.746 46.736) (width 0.25) (layer F.Cu) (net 2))
 (segment (start 126.746 46.736) (end 126.746 41.148) (width 0.25) (layer F.Cu) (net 2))
 (segment (start 104.16499 55.85501) (end 104.14 55.88) (width 0.25) (layer F.Cu) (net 6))
 (segment (start 113.03 49.022) (end 113.03 45.212) (width 0.25) (layer F.Cu) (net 6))
 (segment (start 110.940009 51.111991) (end 113.03 49.022) (width 0.25) (layer F.Cu) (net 6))
 (segment (start 106.622009 51.111991) (end 110.940009 51.111991) (width 0.25) (layer F.Cu) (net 6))
 (segment (start 104.14 53.594) (end 106.622009 51.111991) (width 0.25) (layer F.Cu) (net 6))
 (segment (start 104.14 55.88) (end 104.14 53.594) (width 0.25) (layer F.Cu) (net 6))
 (segment (start 101.346 51.308) (end 103.64 53.602) (width 0.25) (layer F.Cu) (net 7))
 (segment (start 103.64 53.602) (end 103.64 55.88) (width 0.25) (layer F.Cu) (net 7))
 (segment (start 101.346 45.212) (end 101.346 51.308) (width 0.25) (layer F.Cu) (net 7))
 (segment (start 90.17 45.212) (end 90.17 46.482) (width 0.25) (layer F.Cu) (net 8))
 (segment (start 90.17 46.482) (end 95.25 51.562) (width 0.25) (layer F.Cu) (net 8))
 (segment (start 103.14 55.134) (end 103.14 55.88) (width 0.25) (layer F.Cu) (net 8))
 (segment (start 99.568 51.562) (end 103.14 55.134) (width 0.25) (layer F.Cu) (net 8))
 (segment (start 95.25 51.562) (end 99.568 51.562) (width 0.25) (layer F.Cu) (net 8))
 (segment (start 106.68 67.31) (end 105.41 68.58) (width 0.25) (layer F.Cu) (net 9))
 (segment (start 115.57 67.31) (end 106.68 67.31) (width 0.25) (layer F.Cu) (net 9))
 (segment (start 106.68 67.31) (end 106.68 63.754) (width 0.25) (layer F.Cu) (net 9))
 (segment (start 104.64 61.714) (end 104.64 60.28) (width 0.25) (layer F.Cu) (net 9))
 (segment (start 106.68 63.754) (end 104.64 61.714) (width 0.25) (layer F.Cu) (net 9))
 (segment (start 107.41 69.85) (end 106.14 71.12) (width 0.25) (layer F.Cu) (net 10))
 (segment (start 108.204 69.85) (end 108.204 68.326) (width 0.25) (layer F.Cu) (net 10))
 (segment (start 115.57 69.85) (end 108.204 69.85) (width 0.25) (layer F.Cu) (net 10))
 (segment (start 108.204 69.85) (end 107.41 69.85) (width 0.25) (layer F.Cu) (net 10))
 (segment (start 108.204 68.326) (end 108.204 68.326) (width 0.25) (layer F.Cu) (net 10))
 (segment (start 108.204 68.326) (end 108.204 68.326) (width 0.25) (layer F.Cu) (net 10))
 (via (at 108.204 68.326) (size 0.8) (drill 0.4) (layers F.Cu B.Cu) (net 10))
 (segment (start 108.204 68.326) (end 108.204 66.294) (width 0.25) (layer B.Cu) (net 10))
 (segment (start 108.204 66.294) (end 108.204 66.294) (width 0.25) (layer B.Cu) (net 10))
 (via (at 108.204 66.294) (size 0.8) (drill 0.4) (layers F.Cu B.Cu) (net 10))
 (segment (start 108.204 66.294) (end 108.204 64.262) (width 0.25) (layer F.Cu) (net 10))
 (segment (start 105.14 61.198) (end 105.14 60.28) (width 0.25) (layer F.Cu) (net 10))
 (segment (start 108.204 64.262) (end 105.14 61.198) (width 0.25) (layer F.Cu) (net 10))
 (segment (start 97.536 58.912) (end 102.854 58.912) (width 0.25) (layer F.Cu) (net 1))
 (segment (start 103.14 59.198) (end 103.14 60.28) (width 0.25) (layer F.Cu) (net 1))
 (segment (start 102.854 58.912) (end 103.14 59.198) (width 0.25) (layer F.Cu) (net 1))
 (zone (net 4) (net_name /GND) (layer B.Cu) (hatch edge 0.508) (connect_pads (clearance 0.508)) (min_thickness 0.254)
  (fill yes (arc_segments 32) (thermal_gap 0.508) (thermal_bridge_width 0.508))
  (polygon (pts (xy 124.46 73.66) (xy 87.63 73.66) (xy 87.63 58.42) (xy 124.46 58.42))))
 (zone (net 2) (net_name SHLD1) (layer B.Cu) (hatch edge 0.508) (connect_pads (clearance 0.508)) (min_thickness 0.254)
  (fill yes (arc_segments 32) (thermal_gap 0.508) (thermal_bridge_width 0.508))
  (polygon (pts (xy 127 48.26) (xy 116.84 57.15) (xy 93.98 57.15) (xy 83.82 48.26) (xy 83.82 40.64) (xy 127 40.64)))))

